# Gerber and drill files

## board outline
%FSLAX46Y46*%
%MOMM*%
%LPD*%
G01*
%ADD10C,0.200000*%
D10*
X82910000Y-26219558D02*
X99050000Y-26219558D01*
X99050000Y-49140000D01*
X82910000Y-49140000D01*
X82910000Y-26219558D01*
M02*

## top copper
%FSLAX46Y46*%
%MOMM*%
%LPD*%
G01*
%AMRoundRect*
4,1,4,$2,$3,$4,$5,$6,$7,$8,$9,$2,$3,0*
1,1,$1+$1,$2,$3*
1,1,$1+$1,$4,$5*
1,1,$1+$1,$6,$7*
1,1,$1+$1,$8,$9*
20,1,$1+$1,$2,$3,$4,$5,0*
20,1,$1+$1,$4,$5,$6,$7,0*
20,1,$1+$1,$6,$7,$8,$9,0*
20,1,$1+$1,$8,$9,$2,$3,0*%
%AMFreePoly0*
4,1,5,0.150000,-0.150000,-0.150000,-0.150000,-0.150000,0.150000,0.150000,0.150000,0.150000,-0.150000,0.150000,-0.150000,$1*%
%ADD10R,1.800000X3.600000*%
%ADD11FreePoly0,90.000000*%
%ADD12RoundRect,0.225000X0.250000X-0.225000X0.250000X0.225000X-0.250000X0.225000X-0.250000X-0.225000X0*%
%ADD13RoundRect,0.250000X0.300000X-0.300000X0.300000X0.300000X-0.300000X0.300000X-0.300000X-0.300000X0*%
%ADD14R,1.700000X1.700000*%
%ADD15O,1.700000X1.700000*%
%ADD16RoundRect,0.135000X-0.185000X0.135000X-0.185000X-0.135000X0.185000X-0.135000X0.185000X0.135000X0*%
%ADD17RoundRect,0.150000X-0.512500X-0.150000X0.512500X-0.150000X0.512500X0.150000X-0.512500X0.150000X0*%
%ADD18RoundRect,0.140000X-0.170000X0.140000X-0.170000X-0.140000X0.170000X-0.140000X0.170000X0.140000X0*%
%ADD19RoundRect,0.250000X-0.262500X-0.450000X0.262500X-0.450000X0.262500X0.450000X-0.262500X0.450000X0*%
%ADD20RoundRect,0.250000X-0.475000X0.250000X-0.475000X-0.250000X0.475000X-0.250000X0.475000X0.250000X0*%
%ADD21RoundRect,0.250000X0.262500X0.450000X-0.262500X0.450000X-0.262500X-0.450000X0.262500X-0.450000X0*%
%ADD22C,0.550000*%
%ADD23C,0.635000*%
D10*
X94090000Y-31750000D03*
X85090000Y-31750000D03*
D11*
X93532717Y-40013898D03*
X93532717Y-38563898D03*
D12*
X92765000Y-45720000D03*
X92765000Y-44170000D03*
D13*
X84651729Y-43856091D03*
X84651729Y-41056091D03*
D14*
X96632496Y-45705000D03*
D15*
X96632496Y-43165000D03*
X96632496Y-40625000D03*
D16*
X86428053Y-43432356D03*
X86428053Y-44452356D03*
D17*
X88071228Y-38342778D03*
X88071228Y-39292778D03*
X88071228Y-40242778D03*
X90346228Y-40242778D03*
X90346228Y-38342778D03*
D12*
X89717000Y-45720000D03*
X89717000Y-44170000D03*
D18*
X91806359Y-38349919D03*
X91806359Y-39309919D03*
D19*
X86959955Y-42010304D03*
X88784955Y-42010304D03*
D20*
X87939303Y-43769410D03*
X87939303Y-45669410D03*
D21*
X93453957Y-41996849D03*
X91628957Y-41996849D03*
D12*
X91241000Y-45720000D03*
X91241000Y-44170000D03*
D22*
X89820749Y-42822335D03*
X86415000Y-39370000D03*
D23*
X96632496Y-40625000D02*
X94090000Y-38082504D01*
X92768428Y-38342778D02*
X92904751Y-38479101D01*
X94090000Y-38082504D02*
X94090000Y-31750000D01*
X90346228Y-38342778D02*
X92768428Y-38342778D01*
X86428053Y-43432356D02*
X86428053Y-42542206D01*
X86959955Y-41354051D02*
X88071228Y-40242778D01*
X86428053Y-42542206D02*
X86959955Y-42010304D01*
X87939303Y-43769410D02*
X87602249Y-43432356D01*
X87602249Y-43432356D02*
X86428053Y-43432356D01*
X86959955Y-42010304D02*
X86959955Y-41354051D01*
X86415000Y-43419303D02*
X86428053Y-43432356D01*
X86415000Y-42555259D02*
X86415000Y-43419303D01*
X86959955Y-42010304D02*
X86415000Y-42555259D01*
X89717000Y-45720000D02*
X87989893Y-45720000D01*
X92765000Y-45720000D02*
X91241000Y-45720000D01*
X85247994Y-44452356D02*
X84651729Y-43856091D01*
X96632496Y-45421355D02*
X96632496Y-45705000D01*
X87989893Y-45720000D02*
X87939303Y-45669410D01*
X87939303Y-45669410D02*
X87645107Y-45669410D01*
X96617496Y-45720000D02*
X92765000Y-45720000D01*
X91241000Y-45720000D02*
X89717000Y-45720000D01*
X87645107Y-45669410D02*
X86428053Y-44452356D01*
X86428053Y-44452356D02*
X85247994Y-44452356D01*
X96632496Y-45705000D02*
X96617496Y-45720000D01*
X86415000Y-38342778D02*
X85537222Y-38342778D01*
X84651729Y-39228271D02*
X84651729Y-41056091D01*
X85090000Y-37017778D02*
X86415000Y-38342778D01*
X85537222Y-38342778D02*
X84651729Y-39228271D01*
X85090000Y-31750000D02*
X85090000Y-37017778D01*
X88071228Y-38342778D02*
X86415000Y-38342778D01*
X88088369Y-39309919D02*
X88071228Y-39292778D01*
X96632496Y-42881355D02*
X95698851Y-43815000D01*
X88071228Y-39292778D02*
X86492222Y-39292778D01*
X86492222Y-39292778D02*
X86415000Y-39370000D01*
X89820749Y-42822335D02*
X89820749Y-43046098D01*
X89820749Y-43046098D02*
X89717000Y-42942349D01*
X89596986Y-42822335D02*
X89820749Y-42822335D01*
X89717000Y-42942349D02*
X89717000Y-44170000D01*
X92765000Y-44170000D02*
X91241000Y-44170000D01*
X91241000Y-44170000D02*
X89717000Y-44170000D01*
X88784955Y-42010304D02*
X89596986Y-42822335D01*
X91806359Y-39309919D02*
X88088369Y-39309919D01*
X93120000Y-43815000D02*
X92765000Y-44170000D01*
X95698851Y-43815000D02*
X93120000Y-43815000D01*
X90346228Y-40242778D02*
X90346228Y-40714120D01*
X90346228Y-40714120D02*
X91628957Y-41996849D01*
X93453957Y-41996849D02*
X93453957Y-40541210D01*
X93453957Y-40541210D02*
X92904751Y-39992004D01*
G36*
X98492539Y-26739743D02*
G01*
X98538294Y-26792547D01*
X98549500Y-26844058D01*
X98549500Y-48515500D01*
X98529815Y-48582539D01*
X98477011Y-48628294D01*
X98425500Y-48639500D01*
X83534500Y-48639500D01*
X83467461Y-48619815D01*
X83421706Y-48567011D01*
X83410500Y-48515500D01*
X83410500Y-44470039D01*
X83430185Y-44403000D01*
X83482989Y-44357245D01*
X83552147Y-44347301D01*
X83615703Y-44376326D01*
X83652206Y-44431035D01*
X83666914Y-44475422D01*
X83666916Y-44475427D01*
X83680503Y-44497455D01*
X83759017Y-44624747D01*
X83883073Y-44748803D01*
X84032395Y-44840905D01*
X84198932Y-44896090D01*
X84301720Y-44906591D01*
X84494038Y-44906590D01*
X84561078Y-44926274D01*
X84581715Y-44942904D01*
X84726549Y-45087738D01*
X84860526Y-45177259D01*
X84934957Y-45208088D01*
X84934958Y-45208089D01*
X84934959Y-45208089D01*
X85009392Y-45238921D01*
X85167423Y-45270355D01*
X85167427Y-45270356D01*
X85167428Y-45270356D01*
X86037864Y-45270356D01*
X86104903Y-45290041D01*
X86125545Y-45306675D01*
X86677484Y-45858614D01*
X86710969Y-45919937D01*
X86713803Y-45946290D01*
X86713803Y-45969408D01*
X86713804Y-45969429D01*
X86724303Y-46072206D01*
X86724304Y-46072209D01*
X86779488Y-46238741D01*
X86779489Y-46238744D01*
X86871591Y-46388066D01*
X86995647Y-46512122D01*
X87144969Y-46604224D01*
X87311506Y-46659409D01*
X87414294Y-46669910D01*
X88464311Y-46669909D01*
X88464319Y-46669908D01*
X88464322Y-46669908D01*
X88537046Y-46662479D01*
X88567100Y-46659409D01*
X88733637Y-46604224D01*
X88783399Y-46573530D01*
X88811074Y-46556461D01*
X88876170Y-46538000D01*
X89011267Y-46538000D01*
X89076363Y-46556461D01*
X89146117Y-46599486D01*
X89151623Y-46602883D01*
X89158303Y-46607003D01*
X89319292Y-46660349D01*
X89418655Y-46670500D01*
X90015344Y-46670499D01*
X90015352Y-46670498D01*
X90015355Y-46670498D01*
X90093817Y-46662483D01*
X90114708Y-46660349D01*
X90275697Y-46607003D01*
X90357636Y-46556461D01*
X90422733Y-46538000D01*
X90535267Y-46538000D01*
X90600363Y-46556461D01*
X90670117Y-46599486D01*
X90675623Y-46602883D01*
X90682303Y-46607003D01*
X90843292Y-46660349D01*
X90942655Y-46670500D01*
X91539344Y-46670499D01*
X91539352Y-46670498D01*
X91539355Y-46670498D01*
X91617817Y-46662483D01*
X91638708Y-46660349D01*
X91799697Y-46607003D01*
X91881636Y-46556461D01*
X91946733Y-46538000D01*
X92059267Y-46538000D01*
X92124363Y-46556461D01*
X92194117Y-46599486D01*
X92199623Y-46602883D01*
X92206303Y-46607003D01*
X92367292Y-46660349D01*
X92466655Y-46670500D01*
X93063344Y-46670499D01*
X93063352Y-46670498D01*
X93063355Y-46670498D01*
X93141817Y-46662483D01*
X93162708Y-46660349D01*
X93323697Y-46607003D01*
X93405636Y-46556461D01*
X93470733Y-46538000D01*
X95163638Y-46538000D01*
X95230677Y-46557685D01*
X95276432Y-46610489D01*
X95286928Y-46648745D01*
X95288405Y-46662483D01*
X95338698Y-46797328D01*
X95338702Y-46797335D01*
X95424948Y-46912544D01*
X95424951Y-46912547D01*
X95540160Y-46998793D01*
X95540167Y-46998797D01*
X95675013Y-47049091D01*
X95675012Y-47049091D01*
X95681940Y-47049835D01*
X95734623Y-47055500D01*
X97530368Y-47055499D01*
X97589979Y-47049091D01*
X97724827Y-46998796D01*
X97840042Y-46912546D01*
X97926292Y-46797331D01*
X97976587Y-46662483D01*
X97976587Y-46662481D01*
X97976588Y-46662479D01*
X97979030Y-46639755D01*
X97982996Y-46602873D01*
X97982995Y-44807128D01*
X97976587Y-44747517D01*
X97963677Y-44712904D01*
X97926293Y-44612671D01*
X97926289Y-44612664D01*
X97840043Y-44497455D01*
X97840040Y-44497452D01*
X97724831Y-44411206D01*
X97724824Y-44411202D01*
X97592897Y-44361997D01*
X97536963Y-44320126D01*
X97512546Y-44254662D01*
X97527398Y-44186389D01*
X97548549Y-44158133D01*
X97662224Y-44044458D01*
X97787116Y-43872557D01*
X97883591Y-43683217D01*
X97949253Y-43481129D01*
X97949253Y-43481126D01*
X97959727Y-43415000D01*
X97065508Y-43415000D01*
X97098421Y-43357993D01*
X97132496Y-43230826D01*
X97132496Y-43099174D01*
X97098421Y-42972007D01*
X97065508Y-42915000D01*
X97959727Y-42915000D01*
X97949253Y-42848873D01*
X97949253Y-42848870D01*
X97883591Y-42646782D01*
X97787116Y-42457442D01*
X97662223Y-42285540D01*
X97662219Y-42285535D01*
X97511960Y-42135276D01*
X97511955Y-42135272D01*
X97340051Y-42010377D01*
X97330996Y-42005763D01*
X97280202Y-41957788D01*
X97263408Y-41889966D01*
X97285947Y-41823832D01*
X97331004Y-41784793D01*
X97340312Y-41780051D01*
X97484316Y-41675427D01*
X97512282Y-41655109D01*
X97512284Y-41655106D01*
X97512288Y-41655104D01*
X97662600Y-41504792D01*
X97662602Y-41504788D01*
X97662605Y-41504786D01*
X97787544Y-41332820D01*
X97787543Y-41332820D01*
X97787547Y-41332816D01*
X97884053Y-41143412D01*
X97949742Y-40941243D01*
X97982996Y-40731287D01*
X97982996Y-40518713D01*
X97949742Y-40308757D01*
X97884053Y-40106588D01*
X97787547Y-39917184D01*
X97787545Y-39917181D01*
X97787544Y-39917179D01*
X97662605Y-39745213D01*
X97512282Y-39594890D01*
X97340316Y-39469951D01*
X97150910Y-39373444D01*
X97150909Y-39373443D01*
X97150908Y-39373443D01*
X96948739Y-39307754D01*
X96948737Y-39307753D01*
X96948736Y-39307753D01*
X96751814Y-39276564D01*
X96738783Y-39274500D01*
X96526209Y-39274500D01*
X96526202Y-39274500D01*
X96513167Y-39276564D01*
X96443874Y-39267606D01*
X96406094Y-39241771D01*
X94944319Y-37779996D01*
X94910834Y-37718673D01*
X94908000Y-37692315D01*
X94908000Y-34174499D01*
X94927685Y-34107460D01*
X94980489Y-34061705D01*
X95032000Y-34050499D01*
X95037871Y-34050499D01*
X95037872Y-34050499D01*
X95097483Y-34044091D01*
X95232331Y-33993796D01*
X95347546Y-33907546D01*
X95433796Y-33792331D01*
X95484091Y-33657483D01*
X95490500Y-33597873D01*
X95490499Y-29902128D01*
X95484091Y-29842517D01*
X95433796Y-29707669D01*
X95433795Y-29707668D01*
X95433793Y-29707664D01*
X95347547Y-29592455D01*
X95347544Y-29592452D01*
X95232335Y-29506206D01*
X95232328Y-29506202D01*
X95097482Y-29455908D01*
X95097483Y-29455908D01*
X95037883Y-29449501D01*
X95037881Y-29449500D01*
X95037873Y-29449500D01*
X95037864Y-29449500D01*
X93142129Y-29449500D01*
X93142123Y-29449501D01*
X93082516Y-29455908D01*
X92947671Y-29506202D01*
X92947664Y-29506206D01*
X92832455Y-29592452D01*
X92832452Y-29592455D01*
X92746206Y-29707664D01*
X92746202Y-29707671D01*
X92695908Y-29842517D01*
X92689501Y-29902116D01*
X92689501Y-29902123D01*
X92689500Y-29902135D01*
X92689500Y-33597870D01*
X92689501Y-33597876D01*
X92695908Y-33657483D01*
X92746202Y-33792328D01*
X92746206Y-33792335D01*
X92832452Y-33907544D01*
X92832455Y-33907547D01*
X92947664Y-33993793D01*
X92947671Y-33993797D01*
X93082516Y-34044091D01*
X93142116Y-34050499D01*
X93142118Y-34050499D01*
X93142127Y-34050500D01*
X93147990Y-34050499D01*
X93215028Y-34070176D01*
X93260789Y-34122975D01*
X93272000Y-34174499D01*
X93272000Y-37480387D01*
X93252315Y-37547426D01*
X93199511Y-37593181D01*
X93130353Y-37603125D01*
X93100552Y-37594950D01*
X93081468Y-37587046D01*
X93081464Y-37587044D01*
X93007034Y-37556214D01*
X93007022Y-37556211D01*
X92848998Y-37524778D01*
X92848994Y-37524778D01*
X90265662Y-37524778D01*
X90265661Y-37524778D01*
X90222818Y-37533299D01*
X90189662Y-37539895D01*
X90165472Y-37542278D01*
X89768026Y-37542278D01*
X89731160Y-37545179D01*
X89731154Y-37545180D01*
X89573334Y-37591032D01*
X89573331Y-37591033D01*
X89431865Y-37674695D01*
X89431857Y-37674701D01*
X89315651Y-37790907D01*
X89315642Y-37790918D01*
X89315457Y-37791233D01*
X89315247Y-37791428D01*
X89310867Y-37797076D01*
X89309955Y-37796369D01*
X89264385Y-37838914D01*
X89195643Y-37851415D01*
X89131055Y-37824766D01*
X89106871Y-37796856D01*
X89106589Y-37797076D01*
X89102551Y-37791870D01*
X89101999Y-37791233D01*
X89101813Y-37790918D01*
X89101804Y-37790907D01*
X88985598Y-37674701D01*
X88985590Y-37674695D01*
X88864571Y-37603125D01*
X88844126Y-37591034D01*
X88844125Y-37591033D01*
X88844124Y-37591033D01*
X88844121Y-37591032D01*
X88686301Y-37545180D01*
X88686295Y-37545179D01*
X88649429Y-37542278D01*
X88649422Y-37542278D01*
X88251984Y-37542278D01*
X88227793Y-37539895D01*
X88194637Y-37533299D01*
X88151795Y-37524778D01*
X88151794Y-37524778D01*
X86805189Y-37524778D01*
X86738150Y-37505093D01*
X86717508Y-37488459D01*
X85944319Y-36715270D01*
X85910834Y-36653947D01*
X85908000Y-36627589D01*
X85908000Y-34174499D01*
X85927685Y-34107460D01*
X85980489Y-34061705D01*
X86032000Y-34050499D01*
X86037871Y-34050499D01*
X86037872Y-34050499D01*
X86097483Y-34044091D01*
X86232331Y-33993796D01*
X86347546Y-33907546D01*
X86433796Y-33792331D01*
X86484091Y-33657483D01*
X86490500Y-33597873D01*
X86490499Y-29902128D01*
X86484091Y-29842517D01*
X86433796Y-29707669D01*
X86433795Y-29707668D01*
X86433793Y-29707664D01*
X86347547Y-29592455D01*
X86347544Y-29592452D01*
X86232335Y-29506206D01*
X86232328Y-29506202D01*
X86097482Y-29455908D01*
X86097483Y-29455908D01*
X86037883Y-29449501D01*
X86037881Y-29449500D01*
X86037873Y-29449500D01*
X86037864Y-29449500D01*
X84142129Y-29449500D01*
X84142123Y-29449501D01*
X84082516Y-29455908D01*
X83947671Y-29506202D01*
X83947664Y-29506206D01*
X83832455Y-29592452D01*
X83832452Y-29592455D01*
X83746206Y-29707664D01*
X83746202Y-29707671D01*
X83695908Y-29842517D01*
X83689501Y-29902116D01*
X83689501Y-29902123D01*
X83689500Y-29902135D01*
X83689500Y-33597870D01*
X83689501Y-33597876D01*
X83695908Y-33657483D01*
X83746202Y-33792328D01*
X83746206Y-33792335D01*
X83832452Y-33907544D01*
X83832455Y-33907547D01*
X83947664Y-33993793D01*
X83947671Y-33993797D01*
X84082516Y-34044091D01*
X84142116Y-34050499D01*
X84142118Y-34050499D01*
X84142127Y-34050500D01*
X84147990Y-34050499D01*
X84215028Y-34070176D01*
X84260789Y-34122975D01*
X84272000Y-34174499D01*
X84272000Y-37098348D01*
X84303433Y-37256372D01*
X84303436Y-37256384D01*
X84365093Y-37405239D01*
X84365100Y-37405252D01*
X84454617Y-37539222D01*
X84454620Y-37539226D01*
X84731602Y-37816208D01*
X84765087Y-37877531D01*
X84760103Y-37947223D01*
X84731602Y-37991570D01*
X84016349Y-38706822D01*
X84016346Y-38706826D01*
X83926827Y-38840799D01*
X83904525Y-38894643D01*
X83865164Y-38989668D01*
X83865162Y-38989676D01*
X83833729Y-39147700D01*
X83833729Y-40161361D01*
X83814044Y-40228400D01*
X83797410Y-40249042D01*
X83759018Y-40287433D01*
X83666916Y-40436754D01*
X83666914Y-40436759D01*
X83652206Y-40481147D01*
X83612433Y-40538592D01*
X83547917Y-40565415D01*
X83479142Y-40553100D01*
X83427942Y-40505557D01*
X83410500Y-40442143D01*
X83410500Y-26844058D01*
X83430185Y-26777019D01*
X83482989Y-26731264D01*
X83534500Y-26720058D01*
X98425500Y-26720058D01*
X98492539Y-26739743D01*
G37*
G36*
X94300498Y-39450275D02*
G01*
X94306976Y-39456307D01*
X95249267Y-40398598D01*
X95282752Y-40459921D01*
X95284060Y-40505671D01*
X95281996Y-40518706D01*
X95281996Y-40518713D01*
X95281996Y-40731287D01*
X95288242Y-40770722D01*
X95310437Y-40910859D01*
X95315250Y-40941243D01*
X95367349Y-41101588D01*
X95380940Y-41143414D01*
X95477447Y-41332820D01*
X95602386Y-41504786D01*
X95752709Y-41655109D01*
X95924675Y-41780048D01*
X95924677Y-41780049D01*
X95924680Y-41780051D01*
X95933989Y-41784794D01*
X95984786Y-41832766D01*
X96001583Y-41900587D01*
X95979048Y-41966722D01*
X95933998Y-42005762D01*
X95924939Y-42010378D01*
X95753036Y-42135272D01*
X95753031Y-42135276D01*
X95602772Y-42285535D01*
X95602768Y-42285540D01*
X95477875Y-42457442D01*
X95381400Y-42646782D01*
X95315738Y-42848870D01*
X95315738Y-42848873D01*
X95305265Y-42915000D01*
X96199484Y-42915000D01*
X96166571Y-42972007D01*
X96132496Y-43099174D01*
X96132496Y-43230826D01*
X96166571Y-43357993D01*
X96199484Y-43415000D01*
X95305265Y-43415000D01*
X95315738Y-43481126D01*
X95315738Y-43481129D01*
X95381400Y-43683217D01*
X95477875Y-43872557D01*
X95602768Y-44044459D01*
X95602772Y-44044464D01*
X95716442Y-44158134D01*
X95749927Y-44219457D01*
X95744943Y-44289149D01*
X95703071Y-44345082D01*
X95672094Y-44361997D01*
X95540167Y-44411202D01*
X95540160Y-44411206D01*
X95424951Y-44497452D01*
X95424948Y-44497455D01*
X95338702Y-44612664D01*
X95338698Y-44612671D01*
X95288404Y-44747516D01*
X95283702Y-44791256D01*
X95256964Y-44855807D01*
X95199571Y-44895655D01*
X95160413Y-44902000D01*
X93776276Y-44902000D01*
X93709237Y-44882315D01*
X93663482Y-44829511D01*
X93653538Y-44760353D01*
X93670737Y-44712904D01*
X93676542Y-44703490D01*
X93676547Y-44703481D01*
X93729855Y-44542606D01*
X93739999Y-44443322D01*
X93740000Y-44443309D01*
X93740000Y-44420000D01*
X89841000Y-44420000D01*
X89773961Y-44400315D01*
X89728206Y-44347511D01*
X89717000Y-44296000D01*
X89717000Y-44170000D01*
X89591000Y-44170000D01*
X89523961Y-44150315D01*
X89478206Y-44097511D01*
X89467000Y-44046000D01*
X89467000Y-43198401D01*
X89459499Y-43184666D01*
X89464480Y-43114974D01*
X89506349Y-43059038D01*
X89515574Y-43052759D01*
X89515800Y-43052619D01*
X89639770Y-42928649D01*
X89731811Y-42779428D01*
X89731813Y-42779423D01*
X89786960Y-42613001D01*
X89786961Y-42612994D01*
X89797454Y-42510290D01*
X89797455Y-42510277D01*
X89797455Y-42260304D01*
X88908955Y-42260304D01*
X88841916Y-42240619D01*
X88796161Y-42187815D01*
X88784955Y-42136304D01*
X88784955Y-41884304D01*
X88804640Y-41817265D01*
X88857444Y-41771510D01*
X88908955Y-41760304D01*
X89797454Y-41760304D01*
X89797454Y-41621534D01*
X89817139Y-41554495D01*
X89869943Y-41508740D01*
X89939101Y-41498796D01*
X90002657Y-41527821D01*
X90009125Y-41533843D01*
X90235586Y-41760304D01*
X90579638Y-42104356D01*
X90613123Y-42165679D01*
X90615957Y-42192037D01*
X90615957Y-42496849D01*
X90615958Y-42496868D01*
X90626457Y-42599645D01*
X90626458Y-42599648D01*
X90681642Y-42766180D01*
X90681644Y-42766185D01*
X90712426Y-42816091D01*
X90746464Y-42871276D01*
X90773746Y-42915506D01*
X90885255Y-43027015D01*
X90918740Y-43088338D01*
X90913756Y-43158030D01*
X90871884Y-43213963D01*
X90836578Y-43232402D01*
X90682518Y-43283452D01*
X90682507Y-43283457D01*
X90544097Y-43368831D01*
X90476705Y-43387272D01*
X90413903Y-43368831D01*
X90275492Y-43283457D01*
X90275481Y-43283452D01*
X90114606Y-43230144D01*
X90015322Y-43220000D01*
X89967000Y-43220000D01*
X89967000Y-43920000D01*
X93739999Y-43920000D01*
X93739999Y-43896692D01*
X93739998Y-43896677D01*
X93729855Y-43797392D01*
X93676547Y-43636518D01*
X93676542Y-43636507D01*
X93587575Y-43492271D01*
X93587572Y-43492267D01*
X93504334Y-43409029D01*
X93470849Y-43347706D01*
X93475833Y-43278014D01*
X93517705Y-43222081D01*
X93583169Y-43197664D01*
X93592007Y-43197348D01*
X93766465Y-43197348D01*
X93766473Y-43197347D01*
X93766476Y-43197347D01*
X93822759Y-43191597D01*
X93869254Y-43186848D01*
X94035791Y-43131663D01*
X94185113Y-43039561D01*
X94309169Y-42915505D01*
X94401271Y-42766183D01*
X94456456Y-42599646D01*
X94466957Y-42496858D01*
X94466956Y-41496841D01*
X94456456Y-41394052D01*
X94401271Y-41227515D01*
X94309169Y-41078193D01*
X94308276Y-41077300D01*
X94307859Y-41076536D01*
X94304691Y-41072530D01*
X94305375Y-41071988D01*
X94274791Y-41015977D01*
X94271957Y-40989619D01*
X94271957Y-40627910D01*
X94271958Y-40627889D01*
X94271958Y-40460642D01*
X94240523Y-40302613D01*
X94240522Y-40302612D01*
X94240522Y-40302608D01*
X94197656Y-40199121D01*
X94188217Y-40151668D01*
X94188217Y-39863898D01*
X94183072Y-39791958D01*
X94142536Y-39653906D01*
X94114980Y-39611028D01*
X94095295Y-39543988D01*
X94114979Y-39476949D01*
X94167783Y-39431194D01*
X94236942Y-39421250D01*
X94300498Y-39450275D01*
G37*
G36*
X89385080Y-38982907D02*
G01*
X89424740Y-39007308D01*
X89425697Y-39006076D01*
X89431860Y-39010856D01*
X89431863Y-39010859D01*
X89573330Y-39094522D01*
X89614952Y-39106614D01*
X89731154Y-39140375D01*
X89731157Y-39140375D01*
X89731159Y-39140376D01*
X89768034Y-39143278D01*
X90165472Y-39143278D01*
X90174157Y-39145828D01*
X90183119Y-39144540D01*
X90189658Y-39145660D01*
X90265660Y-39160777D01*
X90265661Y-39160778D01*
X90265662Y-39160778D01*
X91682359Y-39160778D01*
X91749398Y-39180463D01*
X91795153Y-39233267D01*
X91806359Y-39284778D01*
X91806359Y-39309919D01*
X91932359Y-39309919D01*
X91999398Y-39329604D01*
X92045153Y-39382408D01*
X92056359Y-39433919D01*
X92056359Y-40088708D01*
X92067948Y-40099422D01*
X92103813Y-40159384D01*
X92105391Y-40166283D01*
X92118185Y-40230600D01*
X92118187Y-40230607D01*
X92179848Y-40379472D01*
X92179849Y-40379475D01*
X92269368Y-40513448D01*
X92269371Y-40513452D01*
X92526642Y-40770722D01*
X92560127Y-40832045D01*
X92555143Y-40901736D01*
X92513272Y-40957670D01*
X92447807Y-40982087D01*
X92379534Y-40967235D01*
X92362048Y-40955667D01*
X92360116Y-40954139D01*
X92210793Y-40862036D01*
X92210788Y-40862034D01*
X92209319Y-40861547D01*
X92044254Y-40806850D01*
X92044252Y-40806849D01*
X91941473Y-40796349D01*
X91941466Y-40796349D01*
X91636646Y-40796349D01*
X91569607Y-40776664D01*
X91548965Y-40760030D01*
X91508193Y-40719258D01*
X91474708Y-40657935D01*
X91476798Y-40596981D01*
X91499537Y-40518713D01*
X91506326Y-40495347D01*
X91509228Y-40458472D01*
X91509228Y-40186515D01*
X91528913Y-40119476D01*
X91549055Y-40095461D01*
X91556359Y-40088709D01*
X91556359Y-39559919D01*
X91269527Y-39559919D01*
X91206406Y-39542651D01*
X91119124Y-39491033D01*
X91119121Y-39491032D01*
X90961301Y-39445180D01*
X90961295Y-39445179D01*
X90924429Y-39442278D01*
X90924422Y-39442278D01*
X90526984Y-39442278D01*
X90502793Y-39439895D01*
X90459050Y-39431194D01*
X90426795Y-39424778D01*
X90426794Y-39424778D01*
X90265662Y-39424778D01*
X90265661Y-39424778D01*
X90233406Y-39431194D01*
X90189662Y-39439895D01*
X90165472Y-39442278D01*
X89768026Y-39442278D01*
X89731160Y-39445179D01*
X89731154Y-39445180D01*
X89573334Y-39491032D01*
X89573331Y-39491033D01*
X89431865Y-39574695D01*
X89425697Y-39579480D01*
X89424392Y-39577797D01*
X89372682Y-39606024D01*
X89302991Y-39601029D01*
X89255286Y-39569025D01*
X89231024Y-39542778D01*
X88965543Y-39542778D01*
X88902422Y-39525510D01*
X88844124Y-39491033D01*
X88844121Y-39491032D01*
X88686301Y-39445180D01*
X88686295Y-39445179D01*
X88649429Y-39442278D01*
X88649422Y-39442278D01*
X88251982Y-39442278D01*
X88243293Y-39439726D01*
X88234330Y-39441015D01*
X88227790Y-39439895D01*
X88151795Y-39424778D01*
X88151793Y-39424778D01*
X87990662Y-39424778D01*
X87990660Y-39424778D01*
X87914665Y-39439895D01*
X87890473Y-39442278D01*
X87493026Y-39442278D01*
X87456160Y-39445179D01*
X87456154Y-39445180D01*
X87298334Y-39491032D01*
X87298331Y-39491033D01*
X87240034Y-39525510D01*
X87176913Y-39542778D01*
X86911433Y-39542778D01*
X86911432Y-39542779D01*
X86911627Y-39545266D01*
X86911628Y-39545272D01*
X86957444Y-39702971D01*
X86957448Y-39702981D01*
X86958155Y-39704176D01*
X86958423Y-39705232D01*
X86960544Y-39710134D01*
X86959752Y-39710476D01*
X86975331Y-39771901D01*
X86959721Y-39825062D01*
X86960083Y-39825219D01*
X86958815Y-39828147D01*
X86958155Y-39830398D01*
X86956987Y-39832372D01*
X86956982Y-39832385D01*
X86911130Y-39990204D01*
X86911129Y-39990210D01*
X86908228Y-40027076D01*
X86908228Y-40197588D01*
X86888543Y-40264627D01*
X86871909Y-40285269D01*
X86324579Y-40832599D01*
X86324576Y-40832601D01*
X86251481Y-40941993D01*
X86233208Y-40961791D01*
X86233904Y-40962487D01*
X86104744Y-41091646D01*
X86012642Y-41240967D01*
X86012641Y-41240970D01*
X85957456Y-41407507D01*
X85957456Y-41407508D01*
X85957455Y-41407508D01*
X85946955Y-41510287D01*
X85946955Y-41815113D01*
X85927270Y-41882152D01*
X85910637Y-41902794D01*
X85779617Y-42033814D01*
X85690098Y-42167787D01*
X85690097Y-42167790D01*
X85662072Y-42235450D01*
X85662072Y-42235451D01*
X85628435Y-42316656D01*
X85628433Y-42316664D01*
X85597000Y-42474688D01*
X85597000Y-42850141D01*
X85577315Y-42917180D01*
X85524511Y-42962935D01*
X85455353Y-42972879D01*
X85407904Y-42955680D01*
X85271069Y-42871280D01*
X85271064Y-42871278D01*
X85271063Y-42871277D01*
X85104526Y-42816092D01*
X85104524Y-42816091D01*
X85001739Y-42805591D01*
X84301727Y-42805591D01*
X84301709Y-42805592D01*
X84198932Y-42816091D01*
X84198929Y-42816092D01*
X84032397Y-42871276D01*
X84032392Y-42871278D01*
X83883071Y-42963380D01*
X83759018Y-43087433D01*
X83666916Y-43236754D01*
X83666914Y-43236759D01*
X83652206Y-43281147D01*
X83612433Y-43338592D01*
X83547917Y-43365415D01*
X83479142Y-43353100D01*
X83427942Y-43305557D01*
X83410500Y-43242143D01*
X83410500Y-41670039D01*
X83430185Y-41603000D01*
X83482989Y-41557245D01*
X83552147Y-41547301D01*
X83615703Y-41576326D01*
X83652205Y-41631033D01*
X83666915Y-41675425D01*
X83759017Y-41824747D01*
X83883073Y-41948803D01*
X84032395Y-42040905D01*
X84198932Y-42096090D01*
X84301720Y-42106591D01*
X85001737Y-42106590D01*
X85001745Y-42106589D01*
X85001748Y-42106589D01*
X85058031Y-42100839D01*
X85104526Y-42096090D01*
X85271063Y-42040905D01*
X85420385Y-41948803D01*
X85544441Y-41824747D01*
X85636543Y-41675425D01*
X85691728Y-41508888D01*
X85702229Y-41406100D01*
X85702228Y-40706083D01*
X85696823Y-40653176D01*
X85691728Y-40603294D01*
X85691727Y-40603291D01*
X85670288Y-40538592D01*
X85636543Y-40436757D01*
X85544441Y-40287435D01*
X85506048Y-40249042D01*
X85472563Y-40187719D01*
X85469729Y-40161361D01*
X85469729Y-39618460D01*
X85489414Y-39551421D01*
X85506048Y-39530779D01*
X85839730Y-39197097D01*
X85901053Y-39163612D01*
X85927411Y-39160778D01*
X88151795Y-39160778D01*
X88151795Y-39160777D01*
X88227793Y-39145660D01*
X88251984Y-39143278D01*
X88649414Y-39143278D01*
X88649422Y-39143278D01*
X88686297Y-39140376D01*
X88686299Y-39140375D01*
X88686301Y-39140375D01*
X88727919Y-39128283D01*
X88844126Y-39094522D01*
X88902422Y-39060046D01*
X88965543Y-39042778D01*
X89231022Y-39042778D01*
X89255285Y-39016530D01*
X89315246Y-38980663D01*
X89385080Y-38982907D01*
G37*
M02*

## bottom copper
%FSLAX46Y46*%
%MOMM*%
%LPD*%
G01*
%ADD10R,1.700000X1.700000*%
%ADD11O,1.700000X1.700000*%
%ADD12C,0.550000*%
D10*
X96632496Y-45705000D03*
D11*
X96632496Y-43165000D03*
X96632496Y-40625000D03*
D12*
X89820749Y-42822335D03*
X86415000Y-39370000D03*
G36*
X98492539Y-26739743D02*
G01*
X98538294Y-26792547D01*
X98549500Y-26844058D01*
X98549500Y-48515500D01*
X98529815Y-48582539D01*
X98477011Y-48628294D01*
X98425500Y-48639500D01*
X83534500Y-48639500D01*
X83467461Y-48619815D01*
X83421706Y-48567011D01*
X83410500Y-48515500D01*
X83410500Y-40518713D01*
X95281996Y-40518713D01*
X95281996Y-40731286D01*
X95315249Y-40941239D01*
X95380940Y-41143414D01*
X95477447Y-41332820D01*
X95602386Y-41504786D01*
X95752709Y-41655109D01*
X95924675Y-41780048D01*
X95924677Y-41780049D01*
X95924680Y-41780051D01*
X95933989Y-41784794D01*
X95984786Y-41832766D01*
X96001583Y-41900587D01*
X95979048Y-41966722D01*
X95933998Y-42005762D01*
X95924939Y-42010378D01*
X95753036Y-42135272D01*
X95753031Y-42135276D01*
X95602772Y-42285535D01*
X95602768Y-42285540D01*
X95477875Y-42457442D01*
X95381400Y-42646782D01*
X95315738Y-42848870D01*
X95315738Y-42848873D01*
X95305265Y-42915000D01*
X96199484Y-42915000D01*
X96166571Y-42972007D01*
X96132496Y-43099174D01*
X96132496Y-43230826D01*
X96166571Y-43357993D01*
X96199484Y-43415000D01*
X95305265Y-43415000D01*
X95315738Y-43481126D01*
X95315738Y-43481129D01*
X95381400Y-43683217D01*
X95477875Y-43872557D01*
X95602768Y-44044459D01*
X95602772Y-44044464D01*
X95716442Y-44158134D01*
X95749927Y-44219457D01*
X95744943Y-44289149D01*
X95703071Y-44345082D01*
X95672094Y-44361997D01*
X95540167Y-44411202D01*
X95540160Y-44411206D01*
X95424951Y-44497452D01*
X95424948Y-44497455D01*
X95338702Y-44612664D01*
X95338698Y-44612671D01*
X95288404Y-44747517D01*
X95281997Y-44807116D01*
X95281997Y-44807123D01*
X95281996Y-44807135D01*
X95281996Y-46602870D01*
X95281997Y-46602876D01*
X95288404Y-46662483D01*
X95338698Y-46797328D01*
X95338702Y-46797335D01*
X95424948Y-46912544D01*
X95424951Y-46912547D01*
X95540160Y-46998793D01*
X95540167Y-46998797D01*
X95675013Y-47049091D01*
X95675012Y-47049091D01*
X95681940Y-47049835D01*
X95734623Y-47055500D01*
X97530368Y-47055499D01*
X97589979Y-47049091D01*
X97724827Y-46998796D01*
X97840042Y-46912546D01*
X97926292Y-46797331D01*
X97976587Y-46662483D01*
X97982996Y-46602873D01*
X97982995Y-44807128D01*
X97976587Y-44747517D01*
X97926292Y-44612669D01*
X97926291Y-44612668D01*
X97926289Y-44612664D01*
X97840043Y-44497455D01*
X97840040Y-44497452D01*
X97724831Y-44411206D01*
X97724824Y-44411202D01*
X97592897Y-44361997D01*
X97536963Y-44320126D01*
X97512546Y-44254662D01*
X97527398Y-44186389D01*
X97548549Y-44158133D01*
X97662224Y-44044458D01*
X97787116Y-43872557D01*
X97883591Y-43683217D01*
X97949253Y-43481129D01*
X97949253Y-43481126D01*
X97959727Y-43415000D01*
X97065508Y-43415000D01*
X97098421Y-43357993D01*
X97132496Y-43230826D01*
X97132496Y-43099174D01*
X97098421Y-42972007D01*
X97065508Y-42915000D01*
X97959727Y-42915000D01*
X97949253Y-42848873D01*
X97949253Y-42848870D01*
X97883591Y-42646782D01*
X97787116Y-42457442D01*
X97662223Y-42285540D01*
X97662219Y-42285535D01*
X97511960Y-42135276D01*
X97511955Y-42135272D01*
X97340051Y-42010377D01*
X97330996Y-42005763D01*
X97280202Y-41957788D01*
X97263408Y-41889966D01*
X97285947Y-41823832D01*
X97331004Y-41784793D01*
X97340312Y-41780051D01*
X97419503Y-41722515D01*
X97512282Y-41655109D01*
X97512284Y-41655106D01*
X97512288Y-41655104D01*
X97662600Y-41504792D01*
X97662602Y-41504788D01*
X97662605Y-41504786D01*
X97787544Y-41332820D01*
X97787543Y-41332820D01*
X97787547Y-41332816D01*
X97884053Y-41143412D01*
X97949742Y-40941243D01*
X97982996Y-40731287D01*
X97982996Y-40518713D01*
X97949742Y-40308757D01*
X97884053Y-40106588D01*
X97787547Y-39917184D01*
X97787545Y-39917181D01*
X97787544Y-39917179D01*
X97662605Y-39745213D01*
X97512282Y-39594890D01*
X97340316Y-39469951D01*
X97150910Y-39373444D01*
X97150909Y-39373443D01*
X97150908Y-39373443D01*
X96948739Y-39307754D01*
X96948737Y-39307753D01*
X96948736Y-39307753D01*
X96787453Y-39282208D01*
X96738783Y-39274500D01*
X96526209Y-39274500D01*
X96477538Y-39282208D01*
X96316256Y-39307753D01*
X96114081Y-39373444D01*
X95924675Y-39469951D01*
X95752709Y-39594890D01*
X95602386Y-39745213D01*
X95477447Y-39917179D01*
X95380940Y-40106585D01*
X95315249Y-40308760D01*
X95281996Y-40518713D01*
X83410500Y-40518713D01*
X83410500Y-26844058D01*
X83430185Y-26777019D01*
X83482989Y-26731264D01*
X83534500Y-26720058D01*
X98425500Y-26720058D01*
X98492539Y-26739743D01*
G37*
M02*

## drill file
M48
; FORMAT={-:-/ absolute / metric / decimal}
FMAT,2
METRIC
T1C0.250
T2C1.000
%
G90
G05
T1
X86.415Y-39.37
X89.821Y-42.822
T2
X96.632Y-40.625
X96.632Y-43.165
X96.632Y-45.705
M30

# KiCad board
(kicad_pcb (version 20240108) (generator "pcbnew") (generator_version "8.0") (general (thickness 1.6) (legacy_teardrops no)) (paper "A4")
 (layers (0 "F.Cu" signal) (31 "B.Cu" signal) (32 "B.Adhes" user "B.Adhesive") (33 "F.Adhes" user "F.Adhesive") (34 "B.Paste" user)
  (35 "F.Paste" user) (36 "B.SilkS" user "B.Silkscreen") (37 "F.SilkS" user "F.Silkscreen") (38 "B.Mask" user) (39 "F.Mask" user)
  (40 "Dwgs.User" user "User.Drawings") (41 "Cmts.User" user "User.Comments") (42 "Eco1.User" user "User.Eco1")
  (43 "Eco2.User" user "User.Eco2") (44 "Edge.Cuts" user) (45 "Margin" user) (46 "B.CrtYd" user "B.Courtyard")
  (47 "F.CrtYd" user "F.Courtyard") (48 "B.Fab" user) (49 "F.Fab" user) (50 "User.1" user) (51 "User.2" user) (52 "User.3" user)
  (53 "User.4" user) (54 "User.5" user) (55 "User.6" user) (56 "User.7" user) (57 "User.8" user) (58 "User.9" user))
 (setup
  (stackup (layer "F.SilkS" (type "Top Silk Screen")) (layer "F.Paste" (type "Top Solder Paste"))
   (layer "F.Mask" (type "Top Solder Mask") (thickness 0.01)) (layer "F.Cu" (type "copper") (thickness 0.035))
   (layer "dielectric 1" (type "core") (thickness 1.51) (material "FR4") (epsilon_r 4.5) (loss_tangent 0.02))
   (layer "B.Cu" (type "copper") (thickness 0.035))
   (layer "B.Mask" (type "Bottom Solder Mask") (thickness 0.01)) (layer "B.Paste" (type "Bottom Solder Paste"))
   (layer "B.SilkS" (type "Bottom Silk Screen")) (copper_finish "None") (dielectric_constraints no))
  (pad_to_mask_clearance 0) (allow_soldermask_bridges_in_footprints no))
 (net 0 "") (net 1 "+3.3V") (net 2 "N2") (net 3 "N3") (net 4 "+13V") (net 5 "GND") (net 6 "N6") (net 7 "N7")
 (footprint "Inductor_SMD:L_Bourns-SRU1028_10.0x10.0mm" (layer "F.Cu") (at 89.59 31.75 180)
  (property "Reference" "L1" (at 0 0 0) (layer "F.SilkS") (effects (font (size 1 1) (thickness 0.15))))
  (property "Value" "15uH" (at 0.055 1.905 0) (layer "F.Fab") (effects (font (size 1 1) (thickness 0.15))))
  (pad "1" smd rect (at -4.5 0 180) (size 1.8 3.6) (layers "F.Cu" "F.Paste" "F.Mask") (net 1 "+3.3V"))
  (pad "2" smd rect (at 4.5 0 180) (size 1.8 3.6) (layers "F.Cu" "F.Paste" "F.Mask") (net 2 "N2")))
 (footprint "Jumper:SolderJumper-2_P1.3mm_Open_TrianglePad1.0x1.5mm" (layer "F.Cu") (at 93.532717 39.288898 90)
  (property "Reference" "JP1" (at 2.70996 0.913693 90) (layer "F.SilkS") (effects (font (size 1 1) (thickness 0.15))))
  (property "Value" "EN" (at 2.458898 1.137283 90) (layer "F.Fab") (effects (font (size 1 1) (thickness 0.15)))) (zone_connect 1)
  (pad "1" smd custom (at -0.725 0 90) (size 0.3 0.3) (layers "F.Cu" "F.Mask") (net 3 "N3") (zone_connect 2) (thermal_bridge_angle 45)
   (options (clearance outline) (anchor rect)) (primitives))
  (pad "2" smd custom (at 0.725 0 90) (size 0.3 0.3) (layers "F.Cu" "F.Mask") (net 1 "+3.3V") (zone_connect 2) (thermal_bridge_angle 45)
   (options (clearance outline) (anchor rect)) (primitives)))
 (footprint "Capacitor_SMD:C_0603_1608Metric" (layer "F.Cu") (at 92.765 44.945 90)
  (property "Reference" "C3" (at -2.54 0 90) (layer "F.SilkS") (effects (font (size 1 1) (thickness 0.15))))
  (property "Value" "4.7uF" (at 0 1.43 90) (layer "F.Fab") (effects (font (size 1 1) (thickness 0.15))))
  (pad "1" smd roundrect (at -0.775 0 90) (size 0.9 0.95) (layers "F.Cu" "F.Paste" "F.Mask") (roundrect_rratio 0.25) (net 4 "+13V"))
  (pad "2" smd roundrect (at 0.775 0 90) (size 0.9 0.95) (layers "F.Cu" "F.Paste" "F.Mask") (roundrect_rratio 0.25) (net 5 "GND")))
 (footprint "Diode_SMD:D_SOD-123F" (layer "F.Cu") (at 84.651729 42.456091 90)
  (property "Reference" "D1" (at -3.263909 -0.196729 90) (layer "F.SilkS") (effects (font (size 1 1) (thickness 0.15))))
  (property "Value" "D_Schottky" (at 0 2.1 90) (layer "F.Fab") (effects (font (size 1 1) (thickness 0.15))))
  (pad "1" smd roundrect (at -1.4 0 90) (size 1.1 1.1) (layers "F.Cu" "F.Paste" "F.Mask") (roundrect_rratio 0.2272727273) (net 4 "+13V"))
  (pad "2" smd roundrect (at 1.4 0 90) (size 1.1 1.1) (layers "F.Cu" "F.Paste" "F.Mask") (roundrect_rratio 0.2272727273) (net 2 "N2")))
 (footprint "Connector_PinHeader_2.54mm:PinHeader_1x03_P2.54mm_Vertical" (layer "F.Cu") (at 96.632496 45.705 180)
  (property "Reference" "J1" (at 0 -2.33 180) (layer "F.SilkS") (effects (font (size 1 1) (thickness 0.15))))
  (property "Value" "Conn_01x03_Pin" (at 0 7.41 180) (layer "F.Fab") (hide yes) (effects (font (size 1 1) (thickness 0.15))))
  (pad "1" thru_hole rect (at 0 0 180) (size 1.7 1.7) (drill 1) (layers "*.Cu" "*.Mask") (remove_unused_layers no) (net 4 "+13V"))
  (pad "2" thru_hole oval (at 0 2.54 180) (size 1.7 1.7) (drill 1) (layers "*.Cu" "*.Mask") (remove_unused_layers no) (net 5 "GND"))
  (pad "3" thru_hole oval (at 0 5.08 180) (size 1.7 1.7) (drill 1) (layers "*.Cu" "*.Mask") (remove_unused_layers no) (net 1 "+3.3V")))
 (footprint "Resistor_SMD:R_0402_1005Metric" (layer "F.Cu") (at 86.428053 43.942356 -90)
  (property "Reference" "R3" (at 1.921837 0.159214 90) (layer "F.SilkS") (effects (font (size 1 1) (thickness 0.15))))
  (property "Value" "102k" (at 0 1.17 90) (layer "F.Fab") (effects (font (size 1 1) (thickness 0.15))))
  (pad "1" smd roundrect (at -0.51 0 270) (size 0.54 0.64) (layers "F.Cu" "F.Paste" "F.Mask") (roundrect_rratio 0.25) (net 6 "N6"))
  (pad "2" smd roundrect (at 0.51 0 270) (size 0.54 0.64) (layers "F.Cu" "F.Paste" "F.Mask") (roundrect_rratio 0.25) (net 4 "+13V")))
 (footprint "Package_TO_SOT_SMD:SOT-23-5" (layer "F.Cu") (at 89.208728 39.292778)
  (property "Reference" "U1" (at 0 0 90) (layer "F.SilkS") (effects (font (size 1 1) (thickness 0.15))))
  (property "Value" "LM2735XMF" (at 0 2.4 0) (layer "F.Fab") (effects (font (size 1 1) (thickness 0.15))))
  (pad "1" smd roundrect (at -1.1375 -0.95) (size 1.325 0.6) (layers "F.Cu" "F.Paste" "F.Mask") (roundrect_rratio 0.25) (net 2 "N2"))
  (pad "2" smd roundrect (at -1.1375 0) (size 1.325 0.6) (layers "F.Cu" "F.Paste" "F.Mask") (roundrect_rratio 0.25) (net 5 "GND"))
  (pad "3" smd roundrect (at -1.1375 0.95) (size 1.325 0.6) (layers "F.Cu" "F.Paste" "F.Mask") (roundrect_rratio 0.25) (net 6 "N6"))
  (pad "4" smd roundrect (at 1.1375 0.95) (size 1.325 0.6) (layers "F.Cu" "F.Paste" "F.Mask") (roundrect_rratio 0.25) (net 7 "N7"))
  (pad "5" smd roundrect (at 1.1375 -0.95) (size 1.325 0.6) (layers "F.Cu" "F.Paste" "F.Mask") (roundrect_rratio 0.25) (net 1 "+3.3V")))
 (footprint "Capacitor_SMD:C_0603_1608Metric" (layer "F.Cu") (at 89.717 44.945 90)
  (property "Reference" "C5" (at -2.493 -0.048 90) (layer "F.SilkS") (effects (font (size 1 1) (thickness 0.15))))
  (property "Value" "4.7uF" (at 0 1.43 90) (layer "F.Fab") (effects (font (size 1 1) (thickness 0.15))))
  (pad "1" smd roundrect (at -0.775 0 90) (size 0.9 0.95) (layers "F.Cu" "F.Paste" "F.Mask") (roundrect_rratio 0.25) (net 4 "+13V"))
  (pad "2" smd roundrect (at 0.775 0 90) (size 0.9 0.95) (layers "F.Cu" "F.Paste" "F.Mask") (roundrect_rratio 0.25) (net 5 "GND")))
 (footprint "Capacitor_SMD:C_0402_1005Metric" (layer "F.Cu") (at 91.806359 38.829919 -90)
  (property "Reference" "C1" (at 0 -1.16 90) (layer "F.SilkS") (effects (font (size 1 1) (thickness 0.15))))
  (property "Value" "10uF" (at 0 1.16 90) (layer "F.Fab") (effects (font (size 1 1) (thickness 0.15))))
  (pad "1" smd roundrect (at -0.48 0 270) (size 0.56 0.62) (layers "F.Cu" "F.Paste" "F.Mask") (roundrect_rratio 0.25) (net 1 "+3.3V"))
  (pad "2" smd roundrect (at 0.48 0 270) (size 0.56 0.62) (layers "F.Cu" "F.Paste" "F.Mask") (roundrect_rratio 0.25) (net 5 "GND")))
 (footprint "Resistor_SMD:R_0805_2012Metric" (layer "F.Cu") (at 87.872455 42.010304)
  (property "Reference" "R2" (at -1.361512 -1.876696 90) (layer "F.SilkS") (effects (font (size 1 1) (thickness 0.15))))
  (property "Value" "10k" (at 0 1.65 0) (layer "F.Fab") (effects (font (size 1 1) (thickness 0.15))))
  (pad "1" smd roundrect (at -0.9125 0) (size 1.025 1.4) (layers "F.Cu" "F.Paste" "F.Mask") (roundrect_rratio 0.243902) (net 6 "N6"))
  (pad "2" smd roundrect (at 0.9125 0) (size 1.025 1.4) (layers "F.Cu" "F.Paste" "F.Mask") (roundrect_rratio 0.243902) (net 5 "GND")))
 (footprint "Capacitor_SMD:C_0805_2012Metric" (layer "F.Cu") (at 87.939303 44.71941 -90)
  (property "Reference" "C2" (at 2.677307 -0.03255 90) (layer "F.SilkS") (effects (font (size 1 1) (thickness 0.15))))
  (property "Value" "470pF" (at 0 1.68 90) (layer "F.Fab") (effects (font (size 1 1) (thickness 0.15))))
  (pad "1" smd roundrect (at -0.95 0 270) (size 1 1.45) (layers "F.Cu" "F.Paste" "F.Mask") (roundrect_rratio 0.25) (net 6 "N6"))
  (pad "2" smd roundrect (at 0.95 0 270) (size 1 1.45) (layers "F.Cu" "F.Paste" "F.Mask") (roundrect_rratio 0.25) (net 4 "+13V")))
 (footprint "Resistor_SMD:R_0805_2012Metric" (layer "F.Cu") (at 92.541457 41.996849 180)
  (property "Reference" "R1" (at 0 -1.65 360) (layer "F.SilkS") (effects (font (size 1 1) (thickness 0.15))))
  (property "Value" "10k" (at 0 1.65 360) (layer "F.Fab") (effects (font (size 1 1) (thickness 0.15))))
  (pad "1" smd roundrect (at -0.9125 0 180) (size 1.025 1.4) (layers "F.Cu" "F.Paste" "F.Mask") (roundrect_rratio 0.243902) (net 3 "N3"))
  (pad "2" smd roundrect (at 0.9125 0 180) (size 1.025 1.4) (layers "F.Cu" "F.Paste" "F.Mask") (roundrect_rratio 0.243902) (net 7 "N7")))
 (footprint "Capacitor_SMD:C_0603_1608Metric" (layer "F.Cu") (at 91.241 44.945 90)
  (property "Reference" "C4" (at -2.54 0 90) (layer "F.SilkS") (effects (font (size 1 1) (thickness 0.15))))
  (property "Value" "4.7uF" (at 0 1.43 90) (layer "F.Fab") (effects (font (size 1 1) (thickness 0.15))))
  (pad "1" smd roundrect (at -0.775 0 90) (size 0.9 0.95) (layers "F.Cu" "F.Paste" "F.Mask") (roundrect_rratio 0.25) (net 4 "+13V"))
  (pad "2" smd roundrect (at 0.775 0 90) (size 0.9 0.95) (layers "F.Cu" "F.Paste" "F.Mask") (roundrect_rratio 0.25) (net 5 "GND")))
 (gr_rect (start 82.91 26.219558) (end 99.05 49.14) (stroke (width 0.2) (type default)) (fill none) (layer "Edge.Cuts"))
 (segment (start 96.632496 40.625) (end 94.09 38.082504) (width 0.635) (layer "F.Cu") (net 1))
 (segment (start 92.768428 38.342778) (end 92.904751 38.479101) (width 0.635) (layer "F.Cu") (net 1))
 (segment (start 94.09 38.082504) (end 94.09 31.75) (width 0.635) (layer "F.Cu") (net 1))
 (segment (start 90.346228 38.342778) (end 92.768428 38.342778) (width 0.635) (layer "F.Cu") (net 1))
 (segment (start 86.428053 43.432356) (end 86.428053 42.542206) (width 0.635) (layer "F.Cu") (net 6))
 (segment (start 86.959955 41.354051) (end 88.071228 40.242778) (width 0.635) (layer "F.Cu") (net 6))
 (segment (start 86.428053 42.542206) (end 86.959955 42.010304) (width 0.635) (layer "F.Cu") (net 6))
 (segment (start 87.939303 43.76941) (end 87.602249 43.432356) (width 0.635) (layer "F.Cu") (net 6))
 (segment (start 87.602249 43.432356) (end 86.428053 43.432356) (width 0.635) (layer "F.Cu") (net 6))
 (segment (start 86.959955 42.010304) (end 86.959955 41.354051) (width 0.635) (layer "F.Cu") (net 6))
 (segment (start 86.415 43.419303) (end 86.428053 43.432356) (width 0.635) (layer "F.Cu") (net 6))
 (segment (start 86.415 42.555259) (end 86.415 43.419303) (width 0.635) (layer "F.Cu") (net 6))
 (segment (start 86.959955 42.010304) (end 86.415 42.555259) (width 0.635) (layer "F.Cu") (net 6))
 (segment (start 89.717 45.72) (end 87.989893 45.72) (width 0.635) (layer "F.Cu") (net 4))
 (segment (start 92.765 45.72) (end 91.241 45.72) (width 0.635) (layer "F.Cu") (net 4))
 (segment (start 85.247994 44.452356) (end 84.651729 43.856091) (width 0.635) (layer "F.Cu") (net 4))
 (segment (start 96.632496 45.421355) (end 96.632496 45.705) (width 0.635) (layer "F.Cu") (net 4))
 (segment (start 87.989893 45.72) (end 87.939303 45.66941) (width 0.635) (layer "F.Cu") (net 4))
 (segment (start 87.939303 45.66941) (end 87.645107 45.66941) (width 0.635) (layer "F.Cu") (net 4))
 (segment (start 96.617496 45.72) (end 92.765 45.72) (width 0.635) (layer "F.Cu") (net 4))
 (segment (start 91.241 45.72) (end 89.717 45.72) (width 0.635) (layer "F.Cu") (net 4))
 (segment (start 87.645107 45.66941) (end 86.428053 44.452356) (width 0.635) (layer "F.Cu") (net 4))
 (segment (start 86.428053 44.452356) (end 85.247994 44.452356) (width 0.635) (layer "F.Cu") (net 4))
 (segment (start 96.632496 45.705) (end 96.617496 45.72) (width 0.635) (layer "F.Cu") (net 4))
 (segment (start 86.415 38.342778) (end 85.537222 38.342778) (width 0.635) (layer "F.Cu") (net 2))
 (segment (start 84.651729 39.228271) (end 84.651729 41.056091) (width 0.635) (layer "F.Cu") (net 2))
 (segment (start 85.09 37.017778) (end 86.415 38.342778) (width 0.635) (layer "F.Cu") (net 2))
 (segment (start 85.537222 38.342778) (end 84.651729 39.228271) (width 0.635) (layer "F.Cu") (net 2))
 (segment (start 85.09 31.75) (end 85.09 37.017778) (width 0.635) (layer "F.Cu") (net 2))
 (segment (start 88.071228 38.342778) (end 86.415 38.342778) (width 0.635) (layer "F.Cu") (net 2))
 (segment (start 88.088369 39.309919) (end 88.071228 39.292778) (width 0.635) (layer "F.Cu") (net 5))
 (segment (start 96.632496 42.881355) (end 95.698851 43.815) (width 0.635) (layer "F.Cu") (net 5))
 (segment (start 88.071228 39.292778) (end 86.492222 39.292778) (width 0.635) (layer "F.Cu") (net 5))
 (segment (start 86.492222 39.292778) (end 86.415 39.37) (width 0.635) (layer "F.Cu") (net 5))
 (segment (start 89.820749 42.822335) (end 89.820749 43.046098) (width 0.635) (layer "F.Cu") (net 5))
 (segment (start 89.820749 43.046098) (end 89.717 42.942349) (width 0.635) (layer "F.Cu") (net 5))
 (segment (start 89.596986 42.822335) (end 89.820749 42.822335) (width 0.635) (layer "F.Cu") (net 5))
 (segment (start 89.717 42.942349) (end 89.717 44.17) (width 0.635) (layer "F.Cu") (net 5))
 (segment (start 92.765 44.17) (end 91.241 44.17) (width 0.635) (layer "F.Cu") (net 5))
 (segment (start 91.241 44.17) (end 89.717 44.17) (width 0.635) (layer "F.Cu") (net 5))
 (segment (start 88.784955 42.010304) (end 89.596986 42.822335) (width 0.635) (layer "F.Cu") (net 5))
 (segment (start 91.806359 39.309919) (end 88.088369 39.309919) (width 0.635) (layer "F.Cu") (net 5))
 (segment (start 93.12 43.815) (end 92.765 44.17) (width 0.635) (layer "F.Cu") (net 5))
 (segment (start 95.698851 43.815) (end 93.12 43.815) (width 0.635) (layer "F.Cu") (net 5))
 (via (at 89.820749 42.822335) (size 0.55) (drill 0.25) (layers "F.Cu" "B.Cu") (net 5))
 (via (at 86.415 39.37) (size 0.55) (drill 0.25) (layers "F.Cu" "B.Cu") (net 5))
 (segment (start 90.346228 40.242778) (end 90.346228 40.71412) (width 0.635) (layer "F.Cu") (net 7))
 (segment (start 90.346228 40.71412) (end 91.628957 41.996849) (width 0.635) (layer "F.Cu") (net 7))
 (segment (start 93.453957 41.996849) (end 93.453957 40.54121) (width 0.635) (layer "F.Cu") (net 3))
 (segment (start 93.453957 40.54121) (end 92.904751 39.992004) (width 0.635) (layer "F.Cu") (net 3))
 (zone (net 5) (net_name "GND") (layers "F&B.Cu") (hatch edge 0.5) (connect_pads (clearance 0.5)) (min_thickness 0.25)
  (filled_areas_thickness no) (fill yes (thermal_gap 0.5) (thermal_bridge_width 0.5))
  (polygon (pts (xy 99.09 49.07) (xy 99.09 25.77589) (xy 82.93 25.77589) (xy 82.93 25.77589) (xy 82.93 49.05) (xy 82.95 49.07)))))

